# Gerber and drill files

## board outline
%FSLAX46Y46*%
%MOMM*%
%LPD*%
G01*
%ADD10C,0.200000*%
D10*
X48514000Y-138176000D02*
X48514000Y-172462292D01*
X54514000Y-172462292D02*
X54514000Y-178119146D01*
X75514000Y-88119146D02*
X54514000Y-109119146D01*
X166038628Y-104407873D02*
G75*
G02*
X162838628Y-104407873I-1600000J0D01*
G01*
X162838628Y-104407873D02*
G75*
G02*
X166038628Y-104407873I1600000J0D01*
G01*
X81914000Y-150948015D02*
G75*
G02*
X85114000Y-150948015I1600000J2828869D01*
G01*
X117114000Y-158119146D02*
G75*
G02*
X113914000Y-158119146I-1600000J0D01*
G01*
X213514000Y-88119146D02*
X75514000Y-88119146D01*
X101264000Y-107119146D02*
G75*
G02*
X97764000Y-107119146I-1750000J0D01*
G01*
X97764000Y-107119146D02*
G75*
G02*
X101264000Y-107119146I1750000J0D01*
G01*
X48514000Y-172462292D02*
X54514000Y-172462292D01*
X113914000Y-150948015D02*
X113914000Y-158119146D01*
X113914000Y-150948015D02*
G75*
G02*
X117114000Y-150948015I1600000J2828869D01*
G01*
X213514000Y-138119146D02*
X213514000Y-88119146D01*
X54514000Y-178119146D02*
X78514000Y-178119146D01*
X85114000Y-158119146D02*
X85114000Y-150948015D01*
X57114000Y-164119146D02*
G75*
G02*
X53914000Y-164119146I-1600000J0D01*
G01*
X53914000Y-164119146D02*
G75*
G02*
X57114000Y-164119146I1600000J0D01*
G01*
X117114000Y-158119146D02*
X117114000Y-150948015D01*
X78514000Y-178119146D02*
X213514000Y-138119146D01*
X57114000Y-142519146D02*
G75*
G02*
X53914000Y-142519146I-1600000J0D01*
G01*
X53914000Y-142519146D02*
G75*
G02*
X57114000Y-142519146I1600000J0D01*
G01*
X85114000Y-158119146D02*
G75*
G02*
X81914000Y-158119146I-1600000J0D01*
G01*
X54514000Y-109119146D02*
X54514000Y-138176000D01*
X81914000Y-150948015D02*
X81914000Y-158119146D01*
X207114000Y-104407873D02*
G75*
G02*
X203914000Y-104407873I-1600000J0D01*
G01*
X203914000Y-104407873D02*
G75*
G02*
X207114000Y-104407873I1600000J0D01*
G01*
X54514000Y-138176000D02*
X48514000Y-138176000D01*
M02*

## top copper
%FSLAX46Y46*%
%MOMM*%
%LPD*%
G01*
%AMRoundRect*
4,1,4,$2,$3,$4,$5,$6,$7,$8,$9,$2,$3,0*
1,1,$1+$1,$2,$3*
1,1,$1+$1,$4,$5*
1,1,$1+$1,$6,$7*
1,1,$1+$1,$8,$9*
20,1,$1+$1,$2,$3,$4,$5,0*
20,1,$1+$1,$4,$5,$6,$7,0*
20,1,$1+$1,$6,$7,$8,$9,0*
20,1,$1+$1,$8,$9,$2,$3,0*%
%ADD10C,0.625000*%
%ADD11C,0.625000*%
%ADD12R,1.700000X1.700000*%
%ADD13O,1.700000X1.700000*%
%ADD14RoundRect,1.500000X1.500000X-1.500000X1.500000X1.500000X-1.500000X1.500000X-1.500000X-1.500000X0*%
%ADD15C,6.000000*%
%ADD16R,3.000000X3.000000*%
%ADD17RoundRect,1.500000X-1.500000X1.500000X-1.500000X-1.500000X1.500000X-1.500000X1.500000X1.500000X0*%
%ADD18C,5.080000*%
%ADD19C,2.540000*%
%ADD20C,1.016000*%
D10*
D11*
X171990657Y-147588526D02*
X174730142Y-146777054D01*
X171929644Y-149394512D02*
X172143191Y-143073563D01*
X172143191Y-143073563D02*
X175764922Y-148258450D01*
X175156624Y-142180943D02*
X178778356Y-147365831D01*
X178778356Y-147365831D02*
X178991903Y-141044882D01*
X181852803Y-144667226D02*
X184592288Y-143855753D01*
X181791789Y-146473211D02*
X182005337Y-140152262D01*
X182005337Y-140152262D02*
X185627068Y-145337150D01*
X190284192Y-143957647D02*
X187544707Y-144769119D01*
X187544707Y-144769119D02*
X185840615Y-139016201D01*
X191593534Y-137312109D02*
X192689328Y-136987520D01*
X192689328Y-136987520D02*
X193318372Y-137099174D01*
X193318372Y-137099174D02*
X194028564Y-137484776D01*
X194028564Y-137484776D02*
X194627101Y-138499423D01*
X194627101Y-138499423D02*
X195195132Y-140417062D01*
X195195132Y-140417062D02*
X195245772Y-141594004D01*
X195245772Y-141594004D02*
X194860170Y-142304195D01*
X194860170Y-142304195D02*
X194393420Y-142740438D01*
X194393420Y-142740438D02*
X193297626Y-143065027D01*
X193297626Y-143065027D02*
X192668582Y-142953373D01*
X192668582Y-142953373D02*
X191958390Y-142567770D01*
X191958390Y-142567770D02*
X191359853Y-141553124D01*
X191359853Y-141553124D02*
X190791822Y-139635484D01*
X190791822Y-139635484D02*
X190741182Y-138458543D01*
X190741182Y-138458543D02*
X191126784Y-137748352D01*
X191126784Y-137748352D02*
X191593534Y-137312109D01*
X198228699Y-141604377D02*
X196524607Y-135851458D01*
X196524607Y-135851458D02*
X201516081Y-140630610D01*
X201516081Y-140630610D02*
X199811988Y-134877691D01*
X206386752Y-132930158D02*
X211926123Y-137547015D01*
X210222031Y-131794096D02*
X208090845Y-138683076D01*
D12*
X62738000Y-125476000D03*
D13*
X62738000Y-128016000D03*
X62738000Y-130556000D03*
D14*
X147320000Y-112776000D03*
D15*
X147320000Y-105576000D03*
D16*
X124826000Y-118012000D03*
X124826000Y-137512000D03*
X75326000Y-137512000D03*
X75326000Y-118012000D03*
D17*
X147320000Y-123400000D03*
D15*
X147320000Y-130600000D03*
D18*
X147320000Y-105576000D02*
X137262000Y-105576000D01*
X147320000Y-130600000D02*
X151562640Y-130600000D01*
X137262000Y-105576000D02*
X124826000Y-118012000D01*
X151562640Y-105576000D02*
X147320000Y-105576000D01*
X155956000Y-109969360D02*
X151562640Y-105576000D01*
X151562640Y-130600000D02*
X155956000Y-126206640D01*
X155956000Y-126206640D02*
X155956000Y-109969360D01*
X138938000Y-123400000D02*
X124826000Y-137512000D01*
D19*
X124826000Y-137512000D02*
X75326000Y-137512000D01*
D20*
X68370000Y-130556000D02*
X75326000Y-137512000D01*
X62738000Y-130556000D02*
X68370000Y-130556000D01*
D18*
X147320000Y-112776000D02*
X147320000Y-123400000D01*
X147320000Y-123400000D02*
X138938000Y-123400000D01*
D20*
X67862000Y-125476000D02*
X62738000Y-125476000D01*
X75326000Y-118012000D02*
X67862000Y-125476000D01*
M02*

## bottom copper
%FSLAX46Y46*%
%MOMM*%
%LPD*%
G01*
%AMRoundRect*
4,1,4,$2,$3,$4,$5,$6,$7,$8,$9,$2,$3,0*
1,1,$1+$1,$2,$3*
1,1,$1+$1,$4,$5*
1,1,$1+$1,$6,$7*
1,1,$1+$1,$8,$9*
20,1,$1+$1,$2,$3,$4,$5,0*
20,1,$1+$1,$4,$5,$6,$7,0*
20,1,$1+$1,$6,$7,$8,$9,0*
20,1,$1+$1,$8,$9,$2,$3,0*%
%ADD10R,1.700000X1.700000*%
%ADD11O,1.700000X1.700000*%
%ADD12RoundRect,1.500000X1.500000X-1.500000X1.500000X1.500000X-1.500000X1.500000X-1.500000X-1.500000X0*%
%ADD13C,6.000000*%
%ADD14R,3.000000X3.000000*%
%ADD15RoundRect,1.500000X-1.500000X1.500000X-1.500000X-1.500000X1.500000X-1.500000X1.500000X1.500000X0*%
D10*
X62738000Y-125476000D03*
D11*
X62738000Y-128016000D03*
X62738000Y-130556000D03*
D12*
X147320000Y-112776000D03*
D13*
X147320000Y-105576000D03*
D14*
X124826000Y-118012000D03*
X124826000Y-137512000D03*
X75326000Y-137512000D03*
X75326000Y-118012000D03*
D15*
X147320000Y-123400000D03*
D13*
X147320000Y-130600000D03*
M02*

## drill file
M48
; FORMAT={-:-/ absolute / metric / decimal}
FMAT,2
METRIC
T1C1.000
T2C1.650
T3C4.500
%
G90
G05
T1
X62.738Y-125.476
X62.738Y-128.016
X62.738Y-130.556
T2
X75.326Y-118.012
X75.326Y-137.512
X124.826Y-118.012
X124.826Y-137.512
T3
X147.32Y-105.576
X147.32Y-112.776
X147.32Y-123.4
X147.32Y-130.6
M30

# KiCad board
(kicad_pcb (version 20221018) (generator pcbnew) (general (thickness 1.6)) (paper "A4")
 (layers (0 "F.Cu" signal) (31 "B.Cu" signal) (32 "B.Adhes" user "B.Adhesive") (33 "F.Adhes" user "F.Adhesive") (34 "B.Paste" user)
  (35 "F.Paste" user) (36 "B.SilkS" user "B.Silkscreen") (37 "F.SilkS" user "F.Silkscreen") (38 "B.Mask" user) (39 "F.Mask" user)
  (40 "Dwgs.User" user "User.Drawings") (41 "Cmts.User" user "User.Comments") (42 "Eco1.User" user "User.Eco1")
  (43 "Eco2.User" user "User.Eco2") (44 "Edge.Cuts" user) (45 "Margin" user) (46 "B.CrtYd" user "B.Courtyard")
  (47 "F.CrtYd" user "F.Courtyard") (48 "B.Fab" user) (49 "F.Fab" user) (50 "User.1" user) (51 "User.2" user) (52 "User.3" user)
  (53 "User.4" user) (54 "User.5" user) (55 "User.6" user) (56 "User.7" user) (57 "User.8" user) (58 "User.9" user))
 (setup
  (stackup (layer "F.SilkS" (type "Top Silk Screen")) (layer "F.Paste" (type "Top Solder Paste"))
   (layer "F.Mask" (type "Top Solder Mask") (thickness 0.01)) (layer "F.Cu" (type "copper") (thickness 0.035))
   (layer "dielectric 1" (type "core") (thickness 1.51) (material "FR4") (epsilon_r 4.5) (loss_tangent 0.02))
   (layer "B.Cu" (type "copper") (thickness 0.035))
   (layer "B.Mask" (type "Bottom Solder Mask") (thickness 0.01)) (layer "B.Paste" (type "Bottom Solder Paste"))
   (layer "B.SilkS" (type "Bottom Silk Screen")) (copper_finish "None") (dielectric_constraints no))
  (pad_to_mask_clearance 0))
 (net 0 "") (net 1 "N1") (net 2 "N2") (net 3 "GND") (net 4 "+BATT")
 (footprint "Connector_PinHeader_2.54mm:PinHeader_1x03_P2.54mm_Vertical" (layer "F.Cu") (at 62.738 125.476)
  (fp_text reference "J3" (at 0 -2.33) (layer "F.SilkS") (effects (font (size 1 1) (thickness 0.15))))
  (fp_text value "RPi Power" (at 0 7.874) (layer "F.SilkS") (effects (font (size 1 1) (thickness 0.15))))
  (pad "1" thru_hole rect (at 0 0) (size 1.7 1.7) (drill 1) (layers "*.Cu" "*.Mask") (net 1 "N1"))
  (pad "2" thru_hole oval (at 0 2.54) (size 1.7 1.7) (drill 1) (layers "*.Cu" "*.Mask") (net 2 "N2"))
  (pad "3" thru_hole oval (at 0 5.08) (size 1.7 1.7) (drill 1) (layers "*.Cu" "*.Mask") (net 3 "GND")))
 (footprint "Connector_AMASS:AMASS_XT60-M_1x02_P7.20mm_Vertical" (layer "F.Cu") (at 147.32 112.776 90)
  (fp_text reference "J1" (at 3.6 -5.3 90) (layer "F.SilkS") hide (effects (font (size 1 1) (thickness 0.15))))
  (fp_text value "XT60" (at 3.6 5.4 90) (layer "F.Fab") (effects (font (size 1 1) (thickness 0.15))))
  (pad "1" thru_hole roundrect (at 0 0 90) (size 6 6) (drill 4.5) (layers "*.Cu" "*.Mask") (roundrect_rratio 0.25) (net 3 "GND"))
  (pad "2" thru_hole circle (at 7.2 0 90) (size 6 6) (drill 4.5) (layers "*.Cu" "*.Mask") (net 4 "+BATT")))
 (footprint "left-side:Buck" (layer "B.Cu") (at 100.076 127.762 180)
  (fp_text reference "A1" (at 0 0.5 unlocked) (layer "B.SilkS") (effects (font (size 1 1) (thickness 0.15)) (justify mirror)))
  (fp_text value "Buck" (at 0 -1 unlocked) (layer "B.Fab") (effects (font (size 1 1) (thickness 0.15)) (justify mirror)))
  (pad "1" thru_hole rect (at -24.75 9.75 180) (size 3 3) (drill 1.65) (layers "*.Cu" "*.Mask") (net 4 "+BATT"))
  (pad "2" thru_hole rect (at -24.75 -9.75 180) (size 3 3) (drill 1.65) (layers "*.Cu" "*.Mask") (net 3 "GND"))
  (pad "3" thru_hole rect (at 24.75 -9.75 180) (size 3 3) (drill 1.65) (layers "*.Cu" "*.Mask") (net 3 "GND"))
  (pad "4" thru_hole rect (at 24.75 9.75 180) (size 3 3) (drill 1.65) (layers "*.Cu" "*.Mask") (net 1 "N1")))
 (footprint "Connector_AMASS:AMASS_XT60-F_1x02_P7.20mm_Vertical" (layer "B.Cu") (at 147.32 123.4 -90)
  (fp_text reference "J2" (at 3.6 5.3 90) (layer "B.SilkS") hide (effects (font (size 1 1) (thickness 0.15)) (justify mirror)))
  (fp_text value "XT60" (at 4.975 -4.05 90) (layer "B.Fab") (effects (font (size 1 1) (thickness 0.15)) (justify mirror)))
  (pad "1" thru_hole roundrect (at 0 0 270) (size 6 6) (drill 4.5) (layers "*.Cu" "*.Mask") (roundrect_rratio 0.25) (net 3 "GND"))
  (pad "2" thru_hole circle (at 7.2 0 270) (size 6 6) (drill 4.5) (layers "*.Cu" "*.Mask") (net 4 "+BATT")))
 (gr_line (start 48.514 138.176) (end 48.514 172.462292) (stroke (width 0.2) (type solid)) (layer "Edge.Cuts"))
 (gr_line (start 54.514 172.462292) (end 54.514 178.119146) (stroke (width 0.2) (type solid)) (layer "Edge.Cuts"))
 (gr_line (start 75.514 88.119146) (end 54.514 109.119146) (stroke (width 0.2) (type solid)) (layer "Edge.Cuts"))
 (gr_circle (center 164.438628 104.407873) (end 166.038628 104.407873) (stroke (width 0.2) (type solid)) (fill none) (layer "Edge.Cuts"))
 (gr_arc (start 81.914 150.948015) (mid 83.514 144.869146) (end 85.114 150.948015) (stroke (width 0.2) (type solid)) (layer "Edge.Cuts"))
 (gr_arc (start 117.114 158.119146) (mid 115.514 159.719146) (end 113.914 158.119146) (stroke (width 0.2) (type solid)) (layer "Edge.Cuts"))
 (gr_line (start 213.514 88.119146) (end 75.514 88.119146) (stroke (width 0.2) (type solid)) (layer "Edge.Cuts"))
 (gr_circle (center 99.514 107.119146) (end 101.264 107.119146) (stroke (width 0.2) (type solid)) (fill none) (layer "Edge.Cuts"))
 (gr_line (start 48.514 172.462292) (end 54.514 172.462292) (stroke (width 0.2) (type solid)) (layer "Edge.Cuts"))
 (gr_line (start 113.914 150.948015) (end 113.914 158.119146) (stroke (width 0.2) (type solid)) (layer "Edge.Cuts"))
 (gr_arc (start 113.914 150.948015) (mid 115.514 144.869146) (end 117.114 150.948015) (stroke (width 0.2) (type solid)) (layer "Edge.Cuts"))
 (gr_line (start 213.514 138.119146) (end 213.514 88.119146) (stroke (width 0.2) (type solid)) (layer "Edge.Cuts"))
 (gr_line (start 54.514 178.119146) (end 78.514 178.119146) (stroke (width 0.2) (type solid)) (layer "Edge.Cuts"))
 (gr_line (start 85.114 158.119146) (end 85.114 150.948015) (stroke (width 0.2) (type solid)) (layer "Edge.Cuts"))
 (gr_circle (center 55.514 164.119146) (end 57.114 164.119146) (stroke (width 0.2) (type solid)) (fill none) (layer "Edge.Cuts"))
 (gr_line (start 117.114 158.119146) (end 117.114 150.948015) (stroke (width 0.2) (type solid)) (layer "Edge.Cuts"))
 (gr_line (start 78.514 178.119146) (end 213.514 138.119146) (stroke (width 0.2) (type solid)) (layer "Edge.Cuts"))
 (gr_circle (center 55.514 142.519146) (end 57.114 142.519146) (stroke (width 0.2) (type solid)) (fill none) (layer "Edge.Cuts"))
 (gr_arc (start 85.114 158.119146) (mid 83.514 159.719146) (end 81.914 158.119146) (stroke (width 0.2) (type solid)) (layer "Edge.Cuts"))
 (gr_line (start 54.514 109.119146) (end 54.514 138.176) (stroke (width 0.2) (type solid)) (layer "Edge.Cuts"))
 (gr_line (start 81.914 150.948015) (end 81.914 158.119146) (stroke (width 0.2) (type solid)) (layer "Edge.Cuts"))
 (gr_circle (center 205.514 104.407873) (end 207.114 104.407873) (stroke (width 0.2) (type solid)) (fill none) (layer "Edge.Cuts"))
 (gr_line (start 54.514 138.176) (end 48.514 138.176) (stroke (width 0.2) (type solid)) (layer "Edge.Cuts"))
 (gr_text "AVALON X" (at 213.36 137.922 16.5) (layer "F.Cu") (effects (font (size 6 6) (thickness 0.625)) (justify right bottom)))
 (segment (start 147.32 105.576) (end 137.262 105.576) (width 5.08) (layer "F.Cu") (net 4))
 (segment (start 147.32 130.6) (end 151.56264 130.6) (width 5.08) (layer "F.Cu") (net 4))
 (segment (start 137.262 105.576) (end 124.826 118.012) (width 5.08) (layer "F.Cu") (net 4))
 (segment (start 151.56264 105.576) (end 147.32 105.576) (width 5.08) (layer "F.Cu") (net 4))
 (segment (start 155.956 109.96936) (end 151.56264 105.576) (width 5.08) (layer "F.Cu") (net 4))
 (segment (start 151.56264 130.6) (end 155.956 126.20664) (width 5.08) (layer "F.Cu") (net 4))
 (segment (start 155.956 126.20664) (end 155.956 109.96936) (width 5.08) (layer "F.Cu") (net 4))
 (segment (start 138.938 123.4) (end 124.826 137.512) (width 5.08) (layer "F.Cu") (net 3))
 (segment (start 124.826 137.512) (end 75.326 137.512) (width 2.54) (layer "F.Cu") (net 3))
 (segment (start 68.37 130.556) (end 75.326 137.512) (width 1.016) (layer "F.Cu") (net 3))
 (segment (start 62.738 130.556) (end 68.37 130.556) (width 1.016) (layer "F.Cu") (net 3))
 (segment (start 147.32 112.776) (end 147.32 123.4) (width 5.08) (layer "F.Cu") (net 3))
 (segment (start 147.32 123.4) (end 138.938 123.4) (width 5.08) (layer "F.Cu") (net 3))
 (segment (start 67.862 125.476) (end 62.738 125.476) (width 1.016) (layer "F.Cu") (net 1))
 (segment (start 75.326 118.012) (end 67.862 125.476) (width 1.016) (layer "F.Cu") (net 1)))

